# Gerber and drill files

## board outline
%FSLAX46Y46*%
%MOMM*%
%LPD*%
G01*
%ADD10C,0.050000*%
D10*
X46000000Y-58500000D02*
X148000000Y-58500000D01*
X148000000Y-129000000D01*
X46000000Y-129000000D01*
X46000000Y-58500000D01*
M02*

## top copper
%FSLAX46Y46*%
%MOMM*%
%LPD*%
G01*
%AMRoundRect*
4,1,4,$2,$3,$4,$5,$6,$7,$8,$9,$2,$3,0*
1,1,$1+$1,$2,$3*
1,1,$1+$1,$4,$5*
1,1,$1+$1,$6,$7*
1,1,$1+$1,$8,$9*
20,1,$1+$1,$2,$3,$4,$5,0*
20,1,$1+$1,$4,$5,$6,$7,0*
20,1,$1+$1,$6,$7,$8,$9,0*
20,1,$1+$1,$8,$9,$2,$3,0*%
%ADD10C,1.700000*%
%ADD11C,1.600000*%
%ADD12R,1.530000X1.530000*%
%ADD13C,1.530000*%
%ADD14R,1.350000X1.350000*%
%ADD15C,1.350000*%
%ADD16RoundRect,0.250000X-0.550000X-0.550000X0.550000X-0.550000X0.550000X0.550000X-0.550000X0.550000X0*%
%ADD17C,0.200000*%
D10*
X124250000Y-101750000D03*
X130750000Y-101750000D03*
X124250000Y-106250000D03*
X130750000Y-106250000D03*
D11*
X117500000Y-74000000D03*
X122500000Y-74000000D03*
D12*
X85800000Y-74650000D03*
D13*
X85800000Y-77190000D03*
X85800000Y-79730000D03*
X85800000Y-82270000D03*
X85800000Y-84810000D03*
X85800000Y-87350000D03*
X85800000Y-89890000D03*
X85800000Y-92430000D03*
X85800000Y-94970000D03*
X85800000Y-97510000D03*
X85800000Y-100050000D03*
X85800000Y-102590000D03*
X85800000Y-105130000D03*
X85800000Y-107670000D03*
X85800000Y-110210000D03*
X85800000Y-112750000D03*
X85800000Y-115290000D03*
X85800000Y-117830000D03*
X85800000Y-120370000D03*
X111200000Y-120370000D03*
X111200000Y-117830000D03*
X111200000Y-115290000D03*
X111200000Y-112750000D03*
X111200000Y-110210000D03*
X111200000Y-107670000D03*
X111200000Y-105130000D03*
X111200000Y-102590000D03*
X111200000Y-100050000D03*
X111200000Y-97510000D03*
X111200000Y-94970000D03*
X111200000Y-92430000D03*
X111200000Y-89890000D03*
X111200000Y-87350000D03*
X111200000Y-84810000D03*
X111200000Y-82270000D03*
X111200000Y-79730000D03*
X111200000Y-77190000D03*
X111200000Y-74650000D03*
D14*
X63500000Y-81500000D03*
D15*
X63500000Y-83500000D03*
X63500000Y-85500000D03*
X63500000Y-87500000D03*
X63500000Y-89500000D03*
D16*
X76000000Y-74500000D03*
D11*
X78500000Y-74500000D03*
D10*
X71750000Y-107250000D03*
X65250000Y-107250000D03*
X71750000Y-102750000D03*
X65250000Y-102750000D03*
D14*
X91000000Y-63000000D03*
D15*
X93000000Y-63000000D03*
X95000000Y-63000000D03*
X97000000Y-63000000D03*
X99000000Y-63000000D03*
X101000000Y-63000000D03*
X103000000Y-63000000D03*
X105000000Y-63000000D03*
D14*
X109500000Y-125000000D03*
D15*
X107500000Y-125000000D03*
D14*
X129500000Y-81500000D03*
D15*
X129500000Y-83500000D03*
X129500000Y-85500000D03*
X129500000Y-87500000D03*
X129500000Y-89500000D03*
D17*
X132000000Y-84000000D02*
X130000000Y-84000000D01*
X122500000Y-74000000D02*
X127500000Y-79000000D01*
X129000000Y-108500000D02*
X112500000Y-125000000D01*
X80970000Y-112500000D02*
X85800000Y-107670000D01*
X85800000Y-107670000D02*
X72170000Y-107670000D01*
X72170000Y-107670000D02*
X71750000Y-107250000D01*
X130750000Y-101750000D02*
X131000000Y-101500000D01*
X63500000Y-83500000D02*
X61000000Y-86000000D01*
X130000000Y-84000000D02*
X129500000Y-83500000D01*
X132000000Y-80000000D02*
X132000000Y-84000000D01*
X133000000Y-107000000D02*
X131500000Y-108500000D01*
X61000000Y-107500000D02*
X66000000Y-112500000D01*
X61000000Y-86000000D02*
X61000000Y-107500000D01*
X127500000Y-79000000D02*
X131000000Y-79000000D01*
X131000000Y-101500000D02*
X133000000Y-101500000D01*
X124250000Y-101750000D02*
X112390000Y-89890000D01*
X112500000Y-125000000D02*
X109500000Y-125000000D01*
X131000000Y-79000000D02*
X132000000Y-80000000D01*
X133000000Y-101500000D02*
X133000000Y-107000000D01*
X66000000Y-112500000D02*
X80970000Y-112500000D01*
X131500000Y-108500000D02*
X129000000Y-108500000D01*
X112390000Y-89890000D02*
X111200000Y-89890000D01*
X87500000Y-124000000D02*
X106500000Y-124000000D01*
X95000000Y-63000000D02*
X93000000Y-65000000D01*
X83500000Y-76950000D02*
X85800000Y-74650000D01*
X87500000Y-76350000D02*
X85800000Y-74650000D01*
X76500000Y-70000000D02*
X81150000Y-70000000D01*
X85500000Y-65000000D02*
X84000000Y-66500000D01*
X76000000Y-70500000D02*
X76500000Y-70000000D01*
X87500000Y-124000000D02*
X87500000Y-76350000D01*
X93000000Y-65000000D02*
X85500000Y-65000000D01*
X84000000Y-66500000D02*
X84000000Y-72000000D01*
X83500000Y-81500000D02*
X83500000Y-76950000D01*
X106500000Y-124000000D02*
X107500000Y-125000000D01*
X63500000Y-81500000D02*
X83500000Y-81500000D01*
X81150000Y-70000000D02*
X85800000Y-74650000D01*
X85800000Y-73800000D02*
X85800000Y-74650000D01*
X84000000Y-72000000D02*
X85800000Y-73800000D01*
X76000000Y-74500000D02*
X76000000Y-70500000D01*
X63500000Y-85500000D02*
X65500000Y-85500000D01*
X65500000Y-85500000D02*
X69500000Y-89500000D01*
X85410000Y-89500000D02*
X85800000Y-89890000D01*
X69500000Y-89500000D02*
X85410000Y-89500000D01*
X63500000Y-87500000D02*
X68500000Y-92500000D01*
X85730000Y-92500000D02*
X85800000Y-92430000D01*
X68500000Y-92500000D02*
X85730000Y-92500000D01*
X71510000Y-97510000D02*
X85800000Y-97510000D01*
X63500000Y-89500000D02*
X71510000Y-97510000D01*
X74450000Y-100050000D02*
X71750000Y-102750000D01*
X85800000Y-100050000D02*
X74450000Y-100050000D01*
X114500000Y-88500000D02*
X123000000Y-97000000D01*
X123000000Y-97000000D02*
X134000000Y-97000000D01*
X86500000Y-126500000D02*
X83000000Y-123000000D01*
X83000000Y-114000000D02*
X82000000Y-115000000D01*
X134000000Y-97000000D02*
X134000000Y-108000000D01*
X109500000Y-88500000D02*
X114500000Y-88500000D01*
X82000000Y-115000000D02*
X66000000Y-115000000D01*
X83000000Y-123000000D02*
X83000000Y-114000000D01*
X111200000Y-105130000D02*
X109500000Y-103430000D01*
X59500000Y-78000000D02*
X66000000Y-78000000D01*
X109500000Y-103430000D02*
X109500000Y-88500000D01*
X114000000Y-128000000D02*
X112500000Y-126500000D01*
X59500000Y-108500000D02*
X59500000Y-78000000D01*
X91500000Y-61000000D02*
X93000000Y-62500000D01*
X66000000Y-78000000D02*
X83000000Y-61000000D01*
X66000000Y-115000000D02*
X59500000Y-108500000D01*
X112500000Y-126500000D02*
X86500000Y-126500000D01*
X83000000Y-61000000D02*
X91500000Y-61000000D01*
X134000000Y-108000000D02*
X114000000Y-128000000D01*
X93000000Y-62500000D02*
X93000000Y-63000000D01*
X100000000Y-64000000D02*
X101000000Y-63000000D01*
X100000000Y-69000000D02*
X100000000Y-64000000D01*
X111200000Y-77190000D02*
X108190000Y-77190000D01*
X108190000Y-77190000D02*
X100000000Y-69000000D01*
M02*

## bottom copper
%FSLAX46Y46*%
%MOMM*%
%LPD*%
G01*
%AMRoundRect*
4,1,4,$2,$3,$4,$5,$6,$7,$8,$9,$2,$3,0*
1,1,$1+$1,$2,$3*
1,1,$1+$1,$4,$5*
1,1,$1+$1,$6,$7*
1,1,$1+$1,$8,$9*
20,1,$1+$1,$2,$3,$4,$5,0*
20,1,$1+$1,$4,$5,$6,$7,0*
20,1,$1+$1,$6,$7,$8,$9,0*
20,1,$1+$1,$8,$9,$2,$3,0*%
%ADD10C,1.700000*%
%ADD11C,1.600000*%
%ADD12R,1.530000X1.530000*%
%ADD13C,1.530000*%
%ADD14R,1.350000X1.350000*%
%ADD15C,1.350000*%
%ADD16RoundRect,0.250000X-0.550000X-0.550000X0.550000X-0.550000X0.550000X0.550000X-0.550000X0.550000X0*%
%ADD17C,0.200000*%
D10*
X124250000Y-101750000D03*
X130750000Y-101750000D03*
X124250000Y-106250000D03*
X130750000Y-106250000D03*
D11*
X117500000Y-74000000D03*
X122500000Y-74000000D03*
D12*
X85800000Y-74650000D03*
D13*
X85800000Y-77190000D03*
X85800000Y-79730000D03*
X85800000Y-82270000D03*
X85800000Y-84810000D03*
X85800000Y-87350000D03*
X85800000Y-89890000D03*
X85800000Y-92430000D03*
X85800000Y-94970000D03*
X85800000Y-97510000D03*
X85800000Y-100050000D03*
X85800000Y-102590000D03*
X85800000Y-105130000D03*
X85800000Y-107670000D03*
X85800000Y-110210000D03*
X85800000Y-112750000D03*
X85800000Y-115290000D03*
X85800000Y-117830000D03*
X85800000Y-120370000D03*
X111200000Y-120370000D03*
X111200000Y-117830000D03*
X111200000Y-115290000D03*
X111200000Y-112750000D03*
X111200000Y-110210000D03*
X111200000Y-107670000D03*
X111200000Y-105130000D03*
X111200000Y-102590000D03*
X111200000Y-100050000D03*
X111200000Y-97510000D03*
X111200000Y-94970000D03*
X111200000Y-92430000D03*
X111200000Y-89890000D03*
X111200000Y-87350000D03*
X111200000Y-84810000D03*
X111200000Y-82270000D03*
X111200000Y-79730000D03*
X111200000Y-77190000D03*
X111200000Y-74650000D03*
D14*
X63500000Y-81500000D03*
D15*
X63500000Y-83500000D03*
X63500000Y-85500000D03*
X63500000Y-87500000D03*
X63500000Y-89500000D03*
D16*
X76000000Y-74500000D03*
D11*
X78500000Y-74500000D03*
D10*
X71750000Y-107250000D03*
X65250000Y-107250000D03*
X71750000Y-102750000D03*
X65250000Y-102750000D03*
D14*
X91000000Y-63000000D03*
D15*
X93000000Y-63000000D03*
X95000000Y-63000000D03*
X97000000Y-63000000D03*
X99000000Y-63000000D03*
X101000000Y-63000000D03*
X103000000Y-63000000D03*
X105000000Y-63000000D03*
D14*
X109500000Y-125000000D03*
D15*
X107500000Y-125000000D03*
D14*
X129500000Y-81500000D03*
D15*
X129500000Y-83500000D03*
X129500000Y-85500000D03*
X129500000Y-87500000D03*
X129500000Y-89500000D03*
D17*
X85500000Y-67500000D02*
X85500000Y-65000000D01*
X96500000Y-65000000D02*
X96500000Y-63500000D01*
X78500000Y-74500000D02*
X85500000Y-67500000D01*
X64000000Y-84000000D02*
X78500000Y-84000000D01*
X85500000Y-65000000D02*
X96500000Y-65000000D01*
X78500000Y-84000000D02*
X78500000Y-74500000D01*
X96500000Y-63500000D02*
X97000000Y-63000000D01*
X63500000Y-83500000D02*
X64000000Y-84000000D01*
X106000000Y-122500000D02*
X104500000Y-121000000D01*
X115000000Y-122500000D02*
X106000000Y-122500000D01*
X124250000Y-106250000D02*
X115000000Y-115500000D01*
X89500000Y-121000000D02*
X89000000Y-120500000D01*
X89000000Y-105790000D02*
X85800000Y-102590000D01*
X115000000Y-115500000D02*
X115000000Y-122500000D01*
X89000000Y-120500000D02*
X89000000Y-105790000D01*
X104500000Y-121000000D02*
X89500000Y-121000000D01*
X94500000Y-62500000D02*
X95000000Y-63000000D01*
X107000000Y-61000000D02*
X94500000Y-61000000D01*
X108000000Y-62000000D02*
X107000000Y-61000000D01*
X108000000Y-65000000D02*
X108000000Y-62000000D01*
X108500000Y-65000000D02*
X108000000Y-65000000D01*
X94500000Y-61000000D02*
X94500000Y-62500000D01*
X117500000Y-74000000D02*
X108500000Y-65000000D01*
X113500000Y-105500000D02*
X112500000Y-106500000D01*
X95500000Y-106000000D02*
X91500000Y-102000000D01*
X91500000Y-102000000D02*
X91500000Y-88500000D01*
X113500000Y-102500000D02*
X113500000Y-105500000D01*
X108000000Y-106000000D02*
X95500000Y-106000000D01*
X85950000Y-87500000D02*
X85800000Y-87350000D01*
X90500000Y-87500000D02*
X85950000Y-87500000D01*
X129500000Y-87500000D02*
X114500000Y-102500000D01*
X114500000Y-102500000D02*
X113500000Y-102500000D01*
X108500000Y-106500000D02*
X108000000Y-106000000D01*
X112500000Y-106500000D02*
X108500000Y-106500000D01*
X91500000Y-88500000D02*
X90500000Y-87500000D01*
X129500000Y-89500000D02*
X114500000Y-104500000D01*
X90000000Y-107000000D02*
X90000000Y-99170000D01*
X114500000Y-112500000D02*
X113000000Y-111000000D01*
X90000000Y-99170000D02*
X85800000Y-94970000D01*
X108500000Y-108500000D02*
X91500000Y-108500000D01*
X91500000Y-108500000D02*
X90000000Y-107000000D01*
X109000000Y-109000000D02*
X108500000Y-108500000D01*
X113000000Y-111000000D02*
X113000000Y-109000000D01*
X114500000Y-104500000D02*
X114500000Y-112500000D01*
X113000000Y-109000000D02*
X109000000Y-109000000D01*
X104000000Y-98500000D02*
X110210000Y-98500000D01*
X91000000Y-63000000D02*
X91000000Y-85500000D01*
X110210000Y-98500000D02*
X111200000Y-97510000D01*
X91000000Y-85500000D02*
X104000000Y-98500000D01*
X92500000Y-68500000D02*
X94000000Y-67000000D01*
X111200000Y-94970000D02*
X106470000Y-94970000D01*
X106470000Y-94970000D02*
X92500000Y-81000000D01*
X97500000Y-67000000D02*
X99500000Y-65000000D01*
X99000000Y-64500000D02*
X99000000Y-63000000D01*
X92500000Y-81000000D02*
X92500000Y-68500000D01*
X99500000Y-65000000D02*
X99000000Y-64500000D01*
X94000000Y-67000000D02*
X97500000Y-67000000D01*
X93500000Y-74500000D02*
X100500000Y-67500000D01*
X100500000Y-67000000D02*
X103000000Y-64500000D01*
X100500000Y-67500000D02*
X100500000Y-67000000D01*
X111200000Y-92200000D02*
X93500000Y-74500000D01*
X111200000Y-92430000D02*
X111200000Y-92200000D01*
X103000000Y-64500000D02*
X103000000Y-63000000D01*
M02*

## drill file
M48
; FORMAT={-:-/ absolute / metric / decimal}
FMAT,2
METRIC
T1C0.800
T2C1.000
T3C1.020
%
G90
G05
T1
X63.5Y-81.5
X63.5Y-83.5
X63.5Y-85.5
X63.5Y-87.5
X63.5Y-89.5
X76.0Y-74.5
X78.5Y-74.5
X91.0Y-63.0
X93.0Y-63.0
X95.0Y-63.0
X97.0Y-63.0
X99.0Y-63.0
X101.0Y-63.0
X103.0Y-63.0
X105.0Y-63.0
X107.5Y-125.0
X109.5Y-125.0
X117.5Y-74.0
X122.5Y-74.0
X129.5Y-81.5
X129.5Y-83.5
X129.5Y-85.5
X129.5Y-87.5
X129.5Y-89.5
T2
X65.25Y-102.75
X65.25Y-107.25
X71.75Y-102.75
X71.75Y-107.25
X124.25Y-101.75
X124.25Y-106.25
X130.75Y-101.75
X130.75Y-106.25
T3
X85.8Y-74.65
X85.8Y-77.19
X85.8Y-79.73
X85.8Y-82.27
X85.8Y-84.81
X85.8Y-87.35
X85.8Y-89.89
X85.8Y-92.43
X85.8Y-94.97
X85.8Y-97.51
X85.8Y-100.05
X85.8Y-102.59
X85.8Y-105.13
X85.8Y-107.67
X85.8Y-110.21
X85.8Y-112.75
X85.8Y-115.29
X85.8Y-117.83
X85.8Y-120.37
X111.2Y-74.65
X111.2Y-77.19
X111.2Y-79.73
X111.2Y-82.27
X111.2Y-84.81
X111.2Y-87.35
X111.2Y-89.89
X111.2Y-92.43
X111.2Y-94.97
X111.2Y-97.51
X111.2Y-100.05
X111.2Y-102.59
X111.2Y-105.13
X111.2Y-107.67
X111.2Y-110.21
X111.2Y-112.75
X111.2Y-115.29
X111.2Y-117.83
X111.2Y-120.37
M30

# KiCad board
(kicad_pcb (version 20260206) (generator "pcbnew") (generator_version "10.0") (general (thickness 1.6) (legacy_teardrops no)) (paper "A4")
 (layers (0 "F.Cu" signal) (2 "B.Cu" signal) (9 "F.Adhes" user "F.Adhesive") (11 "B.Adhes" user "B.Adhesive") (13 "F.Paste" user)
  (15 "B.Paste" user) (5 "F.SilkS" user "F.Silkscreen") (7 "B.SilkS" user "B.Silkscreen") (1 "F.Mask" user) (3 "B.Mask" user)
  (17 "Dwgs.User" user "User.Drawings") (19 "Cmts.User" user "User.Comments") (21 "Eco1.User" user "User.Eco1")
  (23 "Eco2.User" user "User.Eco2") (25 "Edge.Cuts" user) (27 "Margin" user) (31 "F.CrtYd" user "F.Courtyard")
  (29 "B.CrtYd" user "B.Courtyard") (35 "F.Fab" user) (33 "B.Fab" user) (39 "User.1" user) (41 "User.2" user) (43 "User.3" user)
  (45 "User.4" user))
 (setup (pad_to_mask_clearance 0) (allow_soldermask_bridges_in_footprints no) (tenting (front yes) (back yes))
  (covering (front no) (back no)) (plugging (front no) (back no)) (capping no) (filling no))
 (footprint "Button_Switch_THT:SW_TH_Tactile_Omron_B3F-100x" (layer "F.Cu") (at 124.25 101.75)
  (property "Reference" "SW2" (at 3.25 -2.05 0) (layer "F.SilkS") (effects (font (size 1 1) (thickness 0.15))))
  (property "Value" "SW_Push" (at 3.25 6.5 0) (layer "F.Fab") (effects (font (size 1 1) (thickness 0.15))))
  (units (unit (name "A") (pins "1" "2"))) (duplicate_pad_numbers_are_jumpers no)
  (pad "1" thru_hole circle (at 0 0) (size 1.7 1.7) (drill 1) (layers "*.Cu" "*.Mask") (remove_unused_layers no) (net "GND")
   (thermal_bridge_angle 90))
  (pad "1" thru_hole circle (at 6.5 0) (size 1.7 1.7) (drill 1) (layers "*.Cu" "*.Mask") (remove_unused_layers no) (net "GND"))
  (pad "2" thru_hole circle (at 0 4.5) (size 1.7 1.7) (drill 1) (layers "*.Cu" "*.Mask") (remove_unused_layers no) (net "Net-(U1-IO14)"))
  (pad "2" thru_hole circle (at 6.5 4.5) (size 1.7 1.7) (drill 1) (layers "*.Cu" "*.Mask") (remove_unused_layers no) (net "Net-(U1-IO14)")))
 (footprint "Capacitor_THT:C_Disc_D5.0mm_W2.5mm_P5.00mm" (layer "F.Cu") (at 117.5 74)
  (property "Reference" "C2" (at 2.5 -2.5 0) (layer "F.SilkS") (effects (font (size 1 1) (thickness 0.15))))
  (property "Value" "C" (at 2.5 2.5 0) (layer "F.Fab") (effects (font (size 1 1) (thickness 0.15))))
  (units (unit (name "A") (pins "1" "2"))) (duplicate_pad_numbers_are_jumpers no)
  (pad "1" thru_hole circle (at 0 0) (size 1.6 1.6) (drill 0.8) (layers "*.Cu" "*.Mask") (remove_unused_layers no) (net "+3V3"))
  (pad "2" thru_hole circle (at 5 0) (size 1.6 1.6) (drill 0.8) (layers "*.Cu" "*.Mask") (remove_unused_layers no) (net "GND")))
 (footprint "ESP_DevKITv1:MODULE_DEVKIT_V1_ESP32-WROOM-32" (layer "F.Cu") (at 98.5 97.5)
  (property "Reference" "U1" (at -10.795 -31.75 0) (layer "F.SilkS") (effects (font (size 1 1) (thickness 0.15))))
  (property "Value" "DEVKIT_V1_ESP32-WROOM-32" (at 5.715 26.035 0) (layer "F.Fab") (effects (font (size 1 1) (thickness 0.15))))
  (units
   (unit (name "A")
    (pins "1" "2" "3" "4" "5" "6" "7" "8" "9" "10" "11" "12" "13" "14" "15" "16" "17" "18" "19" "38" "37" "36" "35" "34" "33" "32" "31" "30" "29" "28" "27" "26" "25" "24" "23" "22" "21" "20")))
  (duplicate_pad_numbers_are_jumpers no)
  (pad "1" thru_hole rect (at -12.7 -22.85) (size 1.53 1.53) (drill 1.02) (layers "*.Cu" "*.Mask") (remove_unused_layers no) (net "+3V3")
   (solder_mask_margin 0.102))
  (pad "2" thru_hole circle (at -12.7 -20.31) (size 1.53 1.53) (drill 1.02) (layers "*.Cu" "*.Mask") (remove_unused_layers no)
   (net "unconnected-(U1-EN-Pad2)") (solder_mask_margin 0.102))
  (pad "3" thru_hole circle (at -12.7 -17.77) (size 1.53 1.53) (drill 1.02) (layers "*.Cu" "*.Mask") (remove_unused_layers no)
   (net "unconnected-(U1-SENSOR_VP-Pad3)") (solder_mask_margin 0.102))
  (pad "4" thru_hole circle (at -12.7 -15.23) (size 1.53 1.53) (drill 1.02) (layers "*.Cu" "*.Mask") (remove_unused_layers no)
   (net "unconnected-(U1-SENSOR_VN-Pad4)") (solder_mask_margin 0.102))
  (pad "5" thru_hole circle (at -12.7 -12.69) (size 1.53 1.53) (drill 1.02) (layers "*.Cu" "*.Mask") (remove_unused_layers no)
   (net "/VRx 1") (solder_mask_margin 0.102))
  (pad "6" thru_hole circle (at -12.7 -10.15) (size 1.53 1.53) (drill 1.02) (layers "*.Cu" "*.Mask") (remove_unused_layers no)
   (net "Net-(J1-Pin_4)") (solder_mask_margin 0.102))
  (pad "7" thru_hole circle (at -12.7 -7.61) (size 1.53 1.53) (drill 1.02) (layers "*.Cu" "*.Mask") (remove_unused_layers no)
   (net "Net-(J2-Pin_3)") (solder_mask_margin 0.102))
  (pad "8" thru_hole circle (at -12.7 -5.07) (size 1.53 1.53) (drill 1.02) (layers "*.Cu" "*.Mask") (remove_unused_layers no)
   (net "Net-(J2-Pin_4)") (solder_mask_margin 0.102))
  (pad "9" thru_hole circle (at -12.7 -2.53) (size 1.53 1.53) (drill 1.02) (layers "*.Cu" "*.Mask") (remove_unused_layers no)
   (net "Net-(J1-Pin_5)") (solder_mask_margin 0.102))
  (pad "10" thru_hole circle (at -12.7 0.01) (size 1.53 1.53) (drill 1.02) (layers "*.Cu" "*.Mask") (remove_unused_layers no)
   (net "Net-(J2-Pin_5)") (solder_mask_margin 0.102))
  (pad "11" thru_hole circle (at -12.7 2.55) (size 1.53 1.53) (drill 1.02) (layers "*.Cu" "*.Mask") (remove_unused_layers no)
   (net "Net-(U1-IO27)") (solder_mask_margin 0.102))
  (pad "12" thru_hole circle (at -12.7 5.09) (size 1.53 1.53) (drill 1.02) (layers "*.Cu" "*.Mask") (remove_unused_layers no)
   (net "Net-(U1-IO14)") (solder_mask_margin 0.102))
  (pad "13" thru_hole circle (at -12.7 7.63) (size 1.53 1.53) (drill 1.02) (layers "*.Cu" "*.Mask") (remove_unused_layers no)
   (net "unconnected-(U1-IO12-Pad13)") (solder_mask_margin 0.102))
  (pad "14" thru_hole circle (at -12.7 10.17) (size 1.53 1.53) (drill 1.02) (layers "*.Cu" "*.Mask") (remove_unused_layers no) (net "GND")
   (solder_mask_margin 0.102))
  (pad "15" thru_hole circle (at -12.7 12.71) (size 1.53 1.53) (drill 1.02) (layers "*.Cu" "*.Mask") (remove_unused_layers no)
   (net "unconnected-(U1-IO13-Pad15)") (solder_mask_margin 0.102))
  (pad "16" thru_hole circle (at -12.7 15.25) (size 1.53 1.53) (drill 1.02) (layers "*.Cu" "*.Mask") (remove_unused_layers no)
   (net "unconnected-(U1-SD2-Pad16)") (solder_mask_margin 0.102))
  (pad "17" thru_hole circle (at -12.7 17.79) (size 1.53 1.53) (drill 1.02) (layers "*.Cu" "*.Mask") (remove_unused_layers no)
   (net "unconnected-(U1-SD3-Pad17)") (solder_mask_margin 0.102))
  (pad "18" thru_hole circle (at -12.7 20.33) (size 1.53 1.53) (drill 1.02) (layers "*.Cu" "*.Mask") (remove_unused_layers no)
   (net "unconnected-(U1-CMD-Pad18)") (solder_mask_margin 0.102))
  (pad "19" thru_hole circle (at -12.7 22.87) (size 1.53 1.53) (drill 1.02) (layers "*.Cu" "*.Mask") (remove_unused_layers no)
   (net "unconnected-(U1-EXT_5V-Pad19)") (solder_mask_margin 0.102))
  (pad "20" thru_hole circle (at 12.7 22.87) (size 1.53 1.53) (drill 1.02) (layers "*.Cu" "*.Mask") (remove_unused_layers no)
   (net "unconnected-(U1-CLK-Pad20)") (solder_mask_margin 0.102))
  (pad "21" thru_hole circle (at 12.7 20.33) (size 1.53 1.53) (drill 1.02) (layers "*.Cu" "*.Mask") (remove_unused_layers no)
   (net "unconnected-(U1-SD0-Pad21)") (solder_mask_margin 0.102))
  (pad "22" thru_hole circle (at 12.7 17.79) (size 1.53 1.53) (drill 1.02) (layers "*.Cu" "*.Mask") (remove_unused_layers no)
   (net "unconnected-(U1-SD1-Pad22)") (solder_mask_margin 0.102))
  (pad "23" thru_hole circle (at 12.7 15.25) (size 1.53 1.53) (drill 1.02) (layers "*.Cu" "*.Mask") (remove_unused_layers no)
   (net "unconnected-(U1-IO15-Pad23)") (solder_mask_margin 0.102))
  (pad "24" thru_hole circle (at 12.7 12.71) (size 1.53 1.53) (drill 1.02) (layers "*.Cu" "*.Mask") (remove_unused_layers no)
   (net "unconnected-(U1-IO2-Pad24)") (solder_mask_margin 0.102))
  (pad "25" thru_hole circle (at 12.7 10.17) (size 1.53 1.53) (drill 1.02) (layers "*.Cu" "*.Mask") (remove_unused_layers no)
   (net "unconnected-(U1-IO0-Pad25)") (solder_mask_margin 0.102))
  (pad "26" thru_hole circle (at 12.7 7.63) (size 1.53 1.53) (drill 1.02) (layers "*.Cu" "*.Mask") (remove_unused_layers no)
   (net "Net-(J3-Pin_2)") (solder_mask_margin 0.102))
  (pad "27" thru_hole circle (at 12.7 5.09) (size 1.53 1.53) (drill 1.02) (layers "*.Cu" "*.Mask") (remove_unused_layers no)
   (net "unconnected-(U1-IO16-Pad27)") (solder_mask_margin 0.102))
  (pad "28" thru_hole circle (at 12.7 2.55) (size 1.53 1.53) (drill 1.02) (layers "*.Cu" "*.Mask") (remove_unused_layers no)
   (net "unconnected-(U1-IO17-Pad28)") (solder_mask_margin 0.102))
  (pad "29" thru_hole circle (at 12.7 0.01) (size 1.53 1.53) (drill 1.02) (layers "*.Cu" "*.Mask") (remove_unused_layers no)
   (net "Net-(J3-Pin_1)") (solder_mask_margin 0.102))
  (pad "30" thru_hole circle (at 12.7 -2.53) (size 1.53 1.53) (drill 1.02) (layers "*.Cu" "*.Mask") (remove_unused_layers no)
   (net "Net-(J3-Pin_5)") (solder_mask_margin 0.102))
  (pad "31" thru_hole circle (at 12.7 -5.07) (size 1.53 1.53) (drill 1.02) (layers "*.Cu" "*.Mask") (remove_unused_layers no)
   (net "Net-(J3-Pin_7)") (solder_mask_margin 0.102))
  (pad "32" thru_hole circle (at 12.7 -7.61) (size 1.53 1.53) (drill 1.02) (layers "*.Cu" "*.Mask") (remove_unused_layers no) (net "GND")
   (solder_mask_margin 0.102))
  (pad "33" thru_hole circle (at 12.7 -10.15) (size 1.53 1.53) (drill 1.02) (layers "*.Cu" "*.Mask") (remove_unused_layers no)
   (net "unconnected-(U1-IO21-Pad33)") (solder_mask_margin 0.102))
  (pad "34" thru_hole circle (at 12.7 -12.69) (size 1.53 1.53) (drill 1.02) (layers "*.Cu" "*.Mask") (remove_unused_layers no)
   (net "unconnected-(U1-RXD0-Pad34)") (solder_mask_margin 0.102))
  (pad "35" thru_hole circle (at 12.7 -15.23) (size 1.53 1.53) (drill 1.02) (layers "*.Cu" "*.Mask") (remove_unused_layers no)
   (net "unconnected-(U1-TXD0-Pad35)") (solder_mask_margin 0.102))
  (pad "36" thru_hole circle (at 12.7 -17.77) (size 1.53 1.53) (drill 1.02) (layers "*.Cu" "*.Mask") (remove_unused_layers no)
   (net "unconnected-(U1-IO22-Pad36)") (solder_mask_margin 0.102))
  (pad "37" thru_hole circle (at 12.7 -20.31) (size 1.53 1.53) (drill 1.02) (layers "*.Cu" "*.Mask") (remove_unused_layers no)
   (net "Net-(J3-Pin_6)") (solder_mask_margin 0.102))
  (pad "38" thru_hole circle (at 12.7 -22.85) (size 1.53 1.53) (drill 1.02) (layers "*.Cu" "*.Mask") (remove_unused_layers no) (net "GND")
   (solder_mask_margin 0.102)))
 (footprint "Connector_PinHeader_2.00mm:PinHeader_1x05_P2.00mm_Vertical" (layer "F.Cu") (at 63.5 81.5)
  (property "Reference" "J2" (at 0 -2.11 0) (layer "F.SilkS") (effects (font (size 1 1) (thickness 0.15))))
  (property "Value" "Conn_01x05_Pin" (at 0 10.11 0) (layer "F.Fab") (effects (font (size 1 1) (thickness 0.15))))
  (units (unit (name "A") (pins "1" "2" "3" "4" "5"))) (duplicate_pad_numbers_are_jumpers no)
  (pad "1" thru_hole rect (at 0 0) (size 1.35 1.35) (drill 0.8) (layers "*.Cu" "*.Mask") (remove_unused_layers no) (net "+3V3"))
  (pad "2" thru_hole circle (at 0 2) (size 1.35 1.35) (drill 0.8) (layers "*.Cu" "*.Mask") (remove_unused_layers no) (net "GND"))
  (pad "3" thru_hole circle (at 0 4) (size 1.35 1.35) (drill 0.8) (layers "*.Cu" "*.Mask") (remove_unused_layers no) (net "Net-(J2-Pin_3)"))
  (pad "4" thru_hole circle (at 0 6) (size 1.35 1.35) (drill 0.8) (layers "*.Cu" "*.Mask") (remove_unused_layers no) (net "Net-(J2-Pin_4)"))
  (pad "5" thru_hole circle (at 0 8) (size 1.35 1.35) (drill 0.8) (layers "*.Cu" "*.Mask") (remove_unused_layers no) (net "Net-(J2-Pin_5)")))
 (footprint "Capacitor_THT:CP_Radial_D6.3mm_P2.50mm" (layer "F.Cu") (at 76 74.5)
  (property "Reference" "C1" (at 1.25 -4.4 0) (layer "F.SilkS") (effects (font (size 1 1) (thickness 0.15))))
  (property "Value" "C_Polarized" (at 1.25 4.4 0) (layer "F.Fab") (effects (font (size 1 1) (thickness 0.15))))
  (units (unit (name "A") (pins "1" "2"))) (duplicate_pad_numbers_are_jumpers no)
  (pad "1" thru_hole roundrect (at 0 0) (size 1.6 1.6) (drill 0.8) (layers "*.Cu" "*.Mask") (remove_unused_layers no)
   (roundrect_rratio 0.15625) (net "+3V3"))
  (pad "2" thru_hole circle (at 2.5 0) (size 1.6 1.6) (drill 0.8) (layers "*.Cu" "*.Mask") (remove_unused_layers no) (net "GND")))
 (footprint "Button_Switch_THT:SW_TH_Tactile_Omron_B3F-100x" (layer "F.Cu") (at 71.75 107.25 180)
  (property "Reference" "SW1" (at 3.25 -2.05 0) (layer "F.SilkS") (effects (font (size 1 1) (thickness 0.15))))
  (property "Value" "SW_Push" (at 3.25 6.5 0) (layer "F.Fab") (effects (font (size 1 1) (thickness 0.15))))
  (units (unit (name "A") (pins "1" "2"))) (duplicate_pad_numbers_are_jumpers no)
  (pad "1" thru_hole circle (at 0 0 180) (size 1.7 1.7) (drill 1) (layers "*.Cu" "*.Mask") (remove_unused_layers no) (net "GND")
   (thermal_bridge_angle 90))
  (pad "1" thru_hole circle (at 6.5 0 180) (size 1.7 1.7) (drill 1) (layers "*.Cu" "*.Mask") (remove_unused_layers no) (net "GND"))
  (pad "2" thru_hole circle (at 0 4.5 180) (size 1.7 1.7) (drill 1) (layers "*.Cu" "*.Mask") (remove_unused_layers no) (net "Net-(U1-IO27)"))
  (pad "2" thru_hole circle (at 6.5 4.5 180) (size 1.7 1.7) (drill 1) (layers "*.Cu" "*.Mask") (remove_unused_layers no)
   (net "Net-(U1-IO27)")))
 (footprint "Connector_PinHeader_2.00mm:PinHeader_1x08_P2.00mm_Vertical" (layer "F.Cu") (at 91 63 90)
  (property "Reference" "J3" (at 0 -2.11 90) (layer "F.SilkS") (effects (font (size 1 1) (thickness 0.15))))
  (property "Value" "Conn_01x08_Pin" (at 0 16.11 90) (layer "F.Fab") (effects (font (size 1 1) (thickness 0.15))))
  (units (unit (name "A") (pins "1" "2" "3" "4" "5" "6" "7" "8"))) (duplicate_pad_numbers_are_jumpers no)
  (pad "1" thru_hole rect (at 0 0 90) (size 1.35 1.35) (drill 0.8) (layers "*.Cu" "*.Mask") (remove_unused_layers no) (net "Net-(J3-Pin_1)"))
  (pad "2" thru_hole circle (at 0 2 90) (size 1.35 1.35) (drill 0.8) (layers "*.Cu" "*.Mask") (remove_unused_layers no)
   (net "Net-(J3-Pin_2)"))
  (pad "3" thru_hole circle (at 0 4 90) (size 1.35 1.35) (drill 0.8) (layers "*.Cu" "*.Mask") (remove_unused_layers no) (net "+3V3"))
  (pad "4" thru_hole circle (at 0 6 90) (size 1.35 1.35) (drill 0.8) (layers "*.Cu" "*.Mask") (remove_unused_layers no) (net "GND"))
  (pad "5" thru_hole circle (at 0 8 90) (size 1.35 1.35) (drill 0.8) (layers "*.Cu" "*.Mask") (remove_unused_layers no)
   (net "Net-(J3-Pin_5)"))
  (pad "6" thru_hole circle (at 0 10 90) (size 1.35 1.35) (drill 0.8) (layers "*.Cu" "*.Mask") (remove_unused_layers no)
   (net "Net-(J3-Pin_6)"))
  (pad "7" thru_hole circle (at 0 12 90) (size 1.35 1.35) (drill 0.8) (layers "*.Cu" "*.Mask") (remove_unused_layers no)
   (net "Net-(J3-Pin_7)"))
  (pad "8" thru_hole circle (at 0 14 90) (size 1.35 1.35) (drill 0.8) (layers "*.Cu" "*.Mask") (remove_unused_layers no)
   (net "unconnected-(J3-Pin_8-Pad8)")))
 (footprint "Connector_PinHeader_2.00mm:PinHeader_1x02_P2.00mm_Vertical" (layer "F.Cu") (at 109.5 125 -90)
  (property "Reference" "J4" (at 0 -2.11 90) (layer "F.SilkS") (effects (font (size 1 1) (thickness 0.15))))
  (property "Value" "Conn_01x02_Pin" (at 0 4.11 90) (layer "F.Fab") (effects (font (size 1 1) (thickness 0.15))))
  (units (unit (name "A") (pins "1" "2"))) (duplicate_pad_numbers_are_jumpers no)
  (pad "1" thru_hole rect (at 0 0 270) (size 1.35 1.35) (drill 0.8) (layers "*.Cu" "*.Mask") (remove_unused_layers no) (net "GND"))
  (pad "2" thru_hole circle (at 0 2 270) (size 1.35 1.35) (drill 0.8) (layers "*.Cu" "*.Mask") (remove_unused_layers no) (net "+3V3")))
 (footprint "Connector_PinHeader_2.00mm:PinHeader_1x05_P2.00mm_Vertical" (layer "F.Cu") (at 129.5 81.5)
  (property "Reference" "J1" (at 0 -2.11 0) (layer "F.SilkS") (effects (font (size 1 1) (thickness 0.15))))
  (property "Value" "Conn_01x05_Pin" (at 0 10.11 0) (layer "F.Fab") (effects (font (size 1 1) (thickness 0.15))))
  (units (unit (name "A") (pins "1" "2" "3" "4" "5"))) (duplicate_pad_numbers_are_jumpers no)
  (pad "1" thru_hole rect (at 0 0) (size 1.35 1.35) (drill 0.8) (layers "*.Cu" "*.Mask") (remove_unused_layers no) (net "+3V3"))
  (pad "2" thru_hole circle (at 0 2) (size 1.35 1.35) (drill 0.8) (layers "*.Cu" "*.Mask") (remove_unused_layers no) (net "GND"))
  (pad "3" thru_hole circle (at 0 4) (size 1.35 1.35) (drill 0.8) (layers "*.Cu" "*.Mask") (remove_unused_layers no) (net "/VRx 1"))
  (pad "4" thru_hole circle (at 0 6) (size 1.35 1.35) (drill 0.8) (layers "*.Cu" "*.Mask") (remove_unused_layers no) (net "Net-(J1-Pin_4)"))
  (pad "5" thru_hole circle (at 0 8) (size 1.35 1.35) (drill 0.8) (layers "*.Cu" "*.Mask") (remove_unused_layers no) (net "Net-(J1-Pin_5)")))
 (gr_rect (start 46 58.5) (end 148 129) (stroke (width 0.05) (type default)) (fill no) (layer "Edge.Cuts"))
 (segment (start 132 84) (end 130 84) (width 0.2) (layer "F.Cu") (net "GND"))
 (segment (start 122.5 74) (end 127.5 79) (width 0.2) (layer "F.Cu") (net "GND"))
 (segment (start 129 108.5) (end 112.5 125) (width 0.2) (layer "F.Cu") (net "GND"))
 (segment (start 80.97 112.5) (end 85.8 107.67) (width 0.2) (layer "F.Cu") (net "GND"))
 (segment (start 85.8 107.67) (end 72.17 107.67) (width 0.2) (layer "F.Cu") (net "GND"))
 (segment (start 72.17 107.67) (end 71.75 107.25) (width 0.2) (layer "F.Cu") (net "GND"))
 (segment (start 130.75 101.75) (end 131 101.5) (width 0.2) (layer "F.Cu") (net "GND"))
 (segment (start 63.5 83.5) (end 61 86) (width 0.2) (layer "F.Cu") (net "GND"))
 (segment (start 130 84) (end 129.5 83.5) (width 0.2) (layer "F.Cu") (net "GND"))
 (segment (start 132 80) (end 132 84) (width 0.2) (layer "F.Cu") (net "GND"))
 (segment (start 133 107) (end 131.5 108.5) (width 0.2) (layer "F.Cu") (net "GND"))
 (segment (start 61 107.5) (end 66 112.5) (width 0.2) (layer "F.Cu") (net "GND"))
 (segment (start 61 86) (end 61 107.5) (width 0.2) (layer "F.Cu") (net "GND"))
 (segment (start 127.5 79) (end 131 79) (width 0.2) (layer "F.Cu") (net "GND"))
 (segment (start 131 101.5) (end 133 101.5) (width 0.2) (layer "F.Cu") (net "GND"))
 (segment (start 124.25 101.75) (end 112.39 89.89) (width 0.2) (layer "F.Cu") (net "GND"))
 (segment (start 112.5 125) (end 109.5 125) (width 0.2) (layer "F.Cu") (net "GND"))
 (segment (start 131 79) (end 132 80) (width 0.2) (layer "F.Cu") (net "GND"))
 (segment (start 133 101.5) (end 133 107) (width 0.2) (layer "F.Cu") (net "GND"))
 (segment (start 66 112.5) (end 80.97 112.5) (width 0.2) (layer "F.Cu") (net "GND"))
 (segment (start 131.5 108.5) (end 129 108.5) (width 0.2) (layer "F.Cu") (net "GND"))
 (segment (start 112.39 89.89) (end 111.2 89.89) (width 0.2) (layer "F.Cu") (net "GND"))
 (segment (start 85.5 67.5) (end 85.5 65) (width 0.2) (layer "B.Cu") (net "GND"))
 (segment (start 96.5 65) (end 96.5 63.5) (width 0.2) (layer "B.Cu") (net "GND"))
 (segment (start 78.5 74.5) (end 85.5 67.5) (width 0.2) (layer "B.Cu") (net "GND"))
 (segment (start 64 84) (end 78.5 84) (width 0.2) (layer "B.Cu") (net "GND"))
 (segment (start 85.5 65) (end 96.5 65) (width 0.2) (layer "B.Cu") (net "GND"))
 (segment (start 78.5 84) (end 78.5 74.5) (width 0.2) (layer "B.Cu") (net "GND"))
 (segment (start 96.5 63.5) (end 97 63) (width 0.2) (layer "B.Cu") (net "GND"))
 (segment (start 63.5 83.5) (end 64 84) (width 0.2) (layer "B.Cu") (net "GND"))
 (segment (start 106 122.5) (end 104.5 121) (width 0.2) (layer "B.Cu") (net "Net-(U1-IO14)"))
 (segment (start 115 122.5) (end 106 122.5) (width 0.2) (layer "B.Cu") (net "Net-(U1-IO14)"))
 (segment (start 124.25 106.25) (end 115 115.5) (width 0.2) (layer "B.Cu") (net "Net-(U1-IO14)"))
 (segment (start 89.5 121) (end 89 120.5) (width 0.2) (layer "B.Cu") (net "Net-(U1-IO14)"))
 (segment (start 89 105.79) (end 85.8 102.59) (width 0.2) (layer "B.Cu") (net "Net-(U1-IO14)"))
 (segment (start 115 115.5) (end 115 122.5) (width 0.2) (layer "B.Cu") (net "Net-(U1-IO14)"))
 (segment (start 89 120.5) (end 89 105.79) (width 0.2) (layer "B.Cu") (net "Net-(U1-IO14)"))
 (segment (start 104.5 121) (end 89.5 121) (width 0.2) (layer "B.Cu") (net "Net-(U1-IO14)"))
 (segment (start 87.5 124) (end 106.5 124) (width 0.2) (layer "F.Cu") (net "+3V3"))
 (segment (start 95 63) (end 93 65) (width 0.2) (layer "F.Cu") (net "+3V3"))
 (segment (start 83.5 76.95) (end 85.8 74.65) (width 0.2) (layer "F.Cu") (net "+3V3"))
 (segment (start 87.5 76.35) (end 85.8 74.65) (width 0.2) (layer "F.Cu") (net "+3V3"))
 (segment (start 76.5 70) (end 81.15 70) (width 0.2) (layer "F.Cu") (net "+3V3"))
 (segment (start 85.5 65) (end 84 66.5) (width 0.2) (layer "F.Cu") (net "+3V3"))
 (segment (start 76 70.5) (end 76.5 70) (width 0.2) (layer "F.Cu") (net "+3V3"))
 (segment (start 87.5 124) (end 87.5 76.35) (width 0.2) (layer "F.Cu") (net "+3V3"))
 (segment (start 93 65) (end 85.5 65) (width 0.2) (layer "F.Cu") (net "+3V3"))
 (segment (start 84 66.5) (end 84 72) (width 0.2) (layer "F.Cu") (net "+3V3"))
 (segment (start 83.5 81.5) (end 83.5 76.95) (width 0.2) (layer "F.Cu") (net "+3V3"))
 (segment (start 106.5 124) (end 107.5 125) (width 0.2) (layer "F.Cu") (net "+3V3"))
 (segment (start 63.5 81.5) (end 83.5 81.5) (width 0.2) (layer "F.Cu") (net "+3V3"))
 (segment (start 81.15 70) (end 85.8 74.65) (width 0.2) (layer "F.Cu") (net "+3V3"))
 (segment (start 85.8 73.8) (end 85.8 74.65) (width 0.2) (layer "F.Cu") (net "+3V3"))
 (segment (start 84 72) (end 85.8 73.8) (width 0.2) (layer "F.Cu") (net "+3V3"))
 (segment (start 76 74.5) (end 76 70.5) (width 0.2) (layer "F.Cu") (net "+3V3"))
 (segment (start 94.5 62.5) (end 95 63) (width 0.2) (layer "B.Cu") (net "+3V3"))
 (segment (start 107 61) (end 94.5 61) (width 0.2) (layer "B.Cu") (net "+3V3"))
 (segment (start 108 62) (end 107 61) (width 0.2) (layer "B.Cu") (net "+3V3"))
 (segment (start 108 65) (end 108 62) (width 0.2) (layer "B.Cu") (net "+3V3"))
 (segment (start 108.5 65) (end 108 65) (width 0.2) (layer "B.Cu") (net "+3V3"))
 (segment (start 94.5 61) (end 94.5 62.5) (width 0.2) (layer "B.Cu") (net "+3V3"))
 (segment (start 117.5 74) (end 108.5 65) (width 0.2) (layer "B.Cu") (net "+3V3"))
 (segment (start 113.5 105.5) (end 112.5 106.5) (width 0.2) (layer "B.Cu") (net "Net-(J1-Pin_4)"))
 (segment (start 95.5 106) (end 91.5 102) (width 0.2) (layer "B.Cu") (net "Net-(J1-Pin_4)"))
 (segment (start 91.5 102) (end 91.5 88.5) (width 0.2) (layer "B.Cu") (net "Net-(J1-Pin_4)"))
 (segment (start 113.5 102.5) (end 113.5 105.5) (width 0.2) (layer "B.Cu") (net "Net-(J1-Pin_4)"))
 (segment (start 108 106) (end 95.5 106) (width 0.2) (layer "B.Cu") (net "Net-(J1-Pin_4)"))
 (segment (start 85.95 87.5) (end 85.8 87.35) (width 0.2) (layer "B.Cu") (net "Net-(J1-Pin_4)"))
 (segment (start 90.5 87.5) (end 85.95 87.5) (width 0.2) (layer "B.Cu") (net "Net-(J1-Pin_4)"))
 (segment (start 129.5 87.5) (end 114.5 102.5) (width 0.2) (layer "B.Cu") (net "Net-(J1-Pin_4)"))
 (segment (start 114.5 102.5) (end 113.5 102.5) (width 0.2) (layer "B.Cu") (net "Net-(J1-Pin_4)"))
 (segment (start 108.5 106.5) (end 108 106) (width 0.2) (layer "B.Cu") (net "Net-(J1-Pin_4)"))
 (segment (start 112.5 106.5) (end 108.5 106.5) (width 0.2) (layer "B.Cu") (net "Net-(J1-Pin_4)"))
 (segment (start 91.5 88.5) (end 90.5 87.5) (width 0.2) (layer "B.Cu") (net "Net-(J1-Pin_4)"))
 (segment (start 63.5 85.5) (end 65.5 85.5) (width 0.2) (layer "F.Cu") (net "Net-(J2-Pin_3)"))
 (segment (start 65.5 85.5) (end 69.5 89.5) (width 0.2) (layer "F.Cu") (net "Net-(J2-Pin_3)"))
 (segment (start 85.41 89.5) (end 85.8 89.89) (width 0.2) (layer "F.Cu") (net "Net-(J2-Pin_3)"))
 (segment (start 69.5 89.5) (end 85.41 89.5) (width 0.2) (layer "F.Cu") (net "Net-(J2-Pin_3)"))
 (segment (start 63.5 87.5) (end 68.5 92.5) (width 0.2) (layer "F.Cu") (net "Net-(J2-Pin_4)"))
 (segment (start 85.73 92.5) (end 85.8 92.43) (width 0.2) (layer "F.Cu") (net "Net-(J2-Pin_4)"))
 (segment (start 68.5 92.5) (end 85.73 92.5) (width 0.2) (layer "F.Cu") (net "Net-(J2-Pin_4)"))
 (segment (start 129.5 89.5) (end 114.5 104.5) (width 0.2) (layer "B.Cu") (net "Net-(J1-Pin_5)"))
 (segment (start 90 107) (end 90 99.17) (width 0.2) (layer "B.Cu") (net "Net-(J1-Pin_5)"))
 (segment (start 114.5 112.5) (end 113 111) (width 0.2) (layer "B.Cu") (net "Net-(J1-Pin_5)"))
 (segment (start 90 99.17) (end 85.8 94.97) (width 0.2) (layer "B.Cu") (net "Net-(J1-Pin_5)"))
 (segment (start 108.5 108.5) (end 91.5 108.5) (width 0.2) (layer "B.Cu") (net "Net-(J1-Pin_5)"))
 (segment (start 91.5 108.5) (end 90 107) (width 0.2) (layer "B.Cu") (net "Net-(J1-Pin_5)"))
 (segment (start 109 109) (end 108.5 108.5) (width 0.2) (layer "B.Cu") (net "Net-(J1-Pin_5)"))
 (segment (start 113 111) (end 113 109) (width 0.2) (layer "B.Cu") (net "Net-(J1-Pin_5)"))
 (segment (start 114.5 104.5) (end 114.5 112.5) (width 0.2) (layer "B.Cu") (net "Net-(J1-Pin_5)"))
 (segment (start 113 109) (end 109 109) (width 0.2) (layer "B.Cu") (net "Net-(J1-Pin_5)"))
 (segment (start 71.51 97.51) (end 85.8 97.51) (width 0.2) (layer "F.Cu") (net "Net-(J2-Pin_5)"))
 (segment (start 63.5 89.5) (end 71.51 97.51) (width 0.2) (layer "F.Cu") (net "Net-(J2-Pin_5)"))
 (segment (start 74.45 100.05) (end 71.75 102.75) (width 0.2) (layer "F.Cu") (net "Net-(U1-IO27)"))
 (segment (start 85.8 100.05) (end 74.45 100.05) (width 0.2) (layer "F.Cu") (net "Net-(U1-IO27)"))
 (segment (start 114.5 88.5) (end 123 97) (width 0.2) (layer "F.Cu") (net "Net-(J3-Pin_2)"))
 (segment (start 123 97) (end 134 97) (width 0.2) (layer "F.Cu") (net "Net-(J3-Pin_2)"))
 (segment (start 86.5 126.5) (end 83 123) (width 0.2) (layer "F.Cu") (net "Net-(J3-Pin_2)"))
 (segment (start 83 114) (end 82 115) (width 0.2) (layer "F.Cu") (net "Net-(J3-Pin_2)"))
 (segment (start 134 97) (end 134 108) (width 0.2) (layer "F.Cu") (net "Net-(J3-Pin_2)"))
 (segment (start 109.5 88.5) (end 114.5 88.5) (width 0.2) (layer "F.Cu") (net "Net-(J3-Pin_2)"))
 (segment (start 82 115) (end 66 115) (width 0.2) (layer "F.Cu") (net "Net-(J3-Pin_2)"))
 (segment (start 83 123) (end 83 114) (width 0.2) (layer "F.Cu") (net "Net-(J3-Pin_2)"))
 (segment (start 111.2 105.13) (end 109.5 103.43) (width 0.2) (layer "F.Cu") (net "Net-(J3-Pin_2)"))
 (segment (start 59.5 78) (end 66 78) (width 0.2) (layer "F.Cu") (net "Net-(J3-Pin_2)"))
 (segment (start 109.5 103.43) (end 109.5 88.5) (width 0.2) (layer "F.Cu") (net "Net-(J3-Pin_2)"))
 (segment (start 114 128) (end 112.5 126.5) (width 0.2) (layer "F.Cu") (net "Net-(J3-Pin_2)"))
 (segment (start 59.5 108.5) (end 59.5 78) (width 0.2) (layer "F.Cu") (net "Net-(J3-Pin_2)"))
 (segment (start 91.5 61) (end 93 62.5) (width 0.2) (layer "F.Cu") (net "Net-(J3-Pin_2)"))
 (segment (start 66 78) (end 83 61) (width 0.2) (layer "F.Cu") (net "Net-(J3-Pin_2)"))
 (segment (start 66 115) (end 59.5 108.5) (width 0.2) (layer "F.Cu") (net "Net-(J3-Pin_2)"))
 (segment (start 112.5 126.5) (end 86.5 126.5) (width 0.2) (layer "F.Cu") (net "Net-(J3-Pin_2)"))
 (segment (start 83 61) (end 91.5 61) (width 0.2) (layer "F.Cu") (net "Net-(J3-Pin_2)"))
 (segment (start 134 108) (end 114 128) (width 0.2) (layer "F.Cu") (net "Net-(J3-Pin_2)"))
 (segment (start 93 62.5) (end 93 63) (width 0.2) (layer "F.Cu") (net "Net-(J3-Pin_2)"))
 (segment (start 104 98.5) (end 110.21 98.5) (width 0.2) (layer "B.Cu") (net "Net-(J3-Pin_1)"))
 (segment (start 91 63) (end 91 85.5) (width 0.2) (layer "B.Cu") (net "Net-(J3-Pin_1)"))
 (segment (start 110.21 98.5) (end 111.2 97.51) (width 0.2) (layer "B.Cu") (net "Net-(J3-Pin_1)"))
 (segment (start 91 85.5) (end 104 98.5) (width 0.2) (layer "B.Cu") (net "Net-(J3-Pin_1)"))
 (segment (start 92.5 68.5) (end 94 67) (width 0.2) (layer "B.Cu") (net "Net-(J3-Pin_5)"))
 (segment (start 111.2 94.97) (end 106.47 94.97) (width 0.2) (layer "B.Cu") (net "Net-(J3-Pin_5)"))
 (segment (start 106.47 94.97) (end 92.5 81) (width 0.2) (layer "B.Cu") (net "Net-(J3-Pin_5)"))
 (segment (start 97.5 67) (end 99.5 65) (width 0.2) (layer "B.Cu") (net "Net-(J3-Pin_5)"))
 (segment (start 99 64.5) (end 99 63) (width 0.2) (layer "B.Cu") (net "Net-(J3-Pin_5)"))
 (segment (start 92.5 81) (end 92.5 68.5) (width 0.2) (layer "B.Cu") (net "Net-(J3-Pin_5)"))
 (segment (start 99.5 65) (end 99 64.5) (width 0.2) (layer "B.Cu") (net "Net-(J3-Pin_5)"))
 (segment (start 94 67) (end 97.5 67) (width 0.2) (layer "B.Cu") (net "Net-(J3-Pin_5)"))
 (segment (start 93.5 74.5) (end 100.5 67.5) (width 0.2) (layer "B.Cu") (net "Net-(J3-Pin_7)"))
 (segment (start 100.5 67) (end 103 64.5) (width 0.2) (layer "B.Cu") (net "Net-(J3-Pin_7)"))
 (segment (start 100.5 67.5) (end 100.5 67) (width 0.2) (layer "B.Cu") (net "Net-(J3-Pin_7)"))
 (segment (start 111.2 92.2) (end 93.5 74.5) (width 0.2) (layer "B.Cu") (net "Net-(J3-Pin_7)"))
 (segment (start 111.2 92.43) (end 111.2 92.2) (width 0.2) (layer "B.Cu") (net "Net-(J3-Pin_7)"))
 (segment (start 103 64.5) (end 103 63) (width 0.2) (layer "B.Cu") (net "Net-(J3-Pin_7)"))
 (segment (start 100 64) (end 101 63) (width 0.2) (layer "F.Cu") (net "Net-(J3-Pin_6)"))
 (segment (start 100 69) (end 100 64) (width 0.2) (layer "F.Cu") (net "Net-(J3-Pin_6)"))
 (segment (start 111.2 77.19) (end 108.19 77.19) (width 0.2) (layer "F.Cu") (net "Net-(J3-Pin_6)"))
 (segment (start 108.19 77.19) (end 100 69) (width 0.2) (layer "F.Cu") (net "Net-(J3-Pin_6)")))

